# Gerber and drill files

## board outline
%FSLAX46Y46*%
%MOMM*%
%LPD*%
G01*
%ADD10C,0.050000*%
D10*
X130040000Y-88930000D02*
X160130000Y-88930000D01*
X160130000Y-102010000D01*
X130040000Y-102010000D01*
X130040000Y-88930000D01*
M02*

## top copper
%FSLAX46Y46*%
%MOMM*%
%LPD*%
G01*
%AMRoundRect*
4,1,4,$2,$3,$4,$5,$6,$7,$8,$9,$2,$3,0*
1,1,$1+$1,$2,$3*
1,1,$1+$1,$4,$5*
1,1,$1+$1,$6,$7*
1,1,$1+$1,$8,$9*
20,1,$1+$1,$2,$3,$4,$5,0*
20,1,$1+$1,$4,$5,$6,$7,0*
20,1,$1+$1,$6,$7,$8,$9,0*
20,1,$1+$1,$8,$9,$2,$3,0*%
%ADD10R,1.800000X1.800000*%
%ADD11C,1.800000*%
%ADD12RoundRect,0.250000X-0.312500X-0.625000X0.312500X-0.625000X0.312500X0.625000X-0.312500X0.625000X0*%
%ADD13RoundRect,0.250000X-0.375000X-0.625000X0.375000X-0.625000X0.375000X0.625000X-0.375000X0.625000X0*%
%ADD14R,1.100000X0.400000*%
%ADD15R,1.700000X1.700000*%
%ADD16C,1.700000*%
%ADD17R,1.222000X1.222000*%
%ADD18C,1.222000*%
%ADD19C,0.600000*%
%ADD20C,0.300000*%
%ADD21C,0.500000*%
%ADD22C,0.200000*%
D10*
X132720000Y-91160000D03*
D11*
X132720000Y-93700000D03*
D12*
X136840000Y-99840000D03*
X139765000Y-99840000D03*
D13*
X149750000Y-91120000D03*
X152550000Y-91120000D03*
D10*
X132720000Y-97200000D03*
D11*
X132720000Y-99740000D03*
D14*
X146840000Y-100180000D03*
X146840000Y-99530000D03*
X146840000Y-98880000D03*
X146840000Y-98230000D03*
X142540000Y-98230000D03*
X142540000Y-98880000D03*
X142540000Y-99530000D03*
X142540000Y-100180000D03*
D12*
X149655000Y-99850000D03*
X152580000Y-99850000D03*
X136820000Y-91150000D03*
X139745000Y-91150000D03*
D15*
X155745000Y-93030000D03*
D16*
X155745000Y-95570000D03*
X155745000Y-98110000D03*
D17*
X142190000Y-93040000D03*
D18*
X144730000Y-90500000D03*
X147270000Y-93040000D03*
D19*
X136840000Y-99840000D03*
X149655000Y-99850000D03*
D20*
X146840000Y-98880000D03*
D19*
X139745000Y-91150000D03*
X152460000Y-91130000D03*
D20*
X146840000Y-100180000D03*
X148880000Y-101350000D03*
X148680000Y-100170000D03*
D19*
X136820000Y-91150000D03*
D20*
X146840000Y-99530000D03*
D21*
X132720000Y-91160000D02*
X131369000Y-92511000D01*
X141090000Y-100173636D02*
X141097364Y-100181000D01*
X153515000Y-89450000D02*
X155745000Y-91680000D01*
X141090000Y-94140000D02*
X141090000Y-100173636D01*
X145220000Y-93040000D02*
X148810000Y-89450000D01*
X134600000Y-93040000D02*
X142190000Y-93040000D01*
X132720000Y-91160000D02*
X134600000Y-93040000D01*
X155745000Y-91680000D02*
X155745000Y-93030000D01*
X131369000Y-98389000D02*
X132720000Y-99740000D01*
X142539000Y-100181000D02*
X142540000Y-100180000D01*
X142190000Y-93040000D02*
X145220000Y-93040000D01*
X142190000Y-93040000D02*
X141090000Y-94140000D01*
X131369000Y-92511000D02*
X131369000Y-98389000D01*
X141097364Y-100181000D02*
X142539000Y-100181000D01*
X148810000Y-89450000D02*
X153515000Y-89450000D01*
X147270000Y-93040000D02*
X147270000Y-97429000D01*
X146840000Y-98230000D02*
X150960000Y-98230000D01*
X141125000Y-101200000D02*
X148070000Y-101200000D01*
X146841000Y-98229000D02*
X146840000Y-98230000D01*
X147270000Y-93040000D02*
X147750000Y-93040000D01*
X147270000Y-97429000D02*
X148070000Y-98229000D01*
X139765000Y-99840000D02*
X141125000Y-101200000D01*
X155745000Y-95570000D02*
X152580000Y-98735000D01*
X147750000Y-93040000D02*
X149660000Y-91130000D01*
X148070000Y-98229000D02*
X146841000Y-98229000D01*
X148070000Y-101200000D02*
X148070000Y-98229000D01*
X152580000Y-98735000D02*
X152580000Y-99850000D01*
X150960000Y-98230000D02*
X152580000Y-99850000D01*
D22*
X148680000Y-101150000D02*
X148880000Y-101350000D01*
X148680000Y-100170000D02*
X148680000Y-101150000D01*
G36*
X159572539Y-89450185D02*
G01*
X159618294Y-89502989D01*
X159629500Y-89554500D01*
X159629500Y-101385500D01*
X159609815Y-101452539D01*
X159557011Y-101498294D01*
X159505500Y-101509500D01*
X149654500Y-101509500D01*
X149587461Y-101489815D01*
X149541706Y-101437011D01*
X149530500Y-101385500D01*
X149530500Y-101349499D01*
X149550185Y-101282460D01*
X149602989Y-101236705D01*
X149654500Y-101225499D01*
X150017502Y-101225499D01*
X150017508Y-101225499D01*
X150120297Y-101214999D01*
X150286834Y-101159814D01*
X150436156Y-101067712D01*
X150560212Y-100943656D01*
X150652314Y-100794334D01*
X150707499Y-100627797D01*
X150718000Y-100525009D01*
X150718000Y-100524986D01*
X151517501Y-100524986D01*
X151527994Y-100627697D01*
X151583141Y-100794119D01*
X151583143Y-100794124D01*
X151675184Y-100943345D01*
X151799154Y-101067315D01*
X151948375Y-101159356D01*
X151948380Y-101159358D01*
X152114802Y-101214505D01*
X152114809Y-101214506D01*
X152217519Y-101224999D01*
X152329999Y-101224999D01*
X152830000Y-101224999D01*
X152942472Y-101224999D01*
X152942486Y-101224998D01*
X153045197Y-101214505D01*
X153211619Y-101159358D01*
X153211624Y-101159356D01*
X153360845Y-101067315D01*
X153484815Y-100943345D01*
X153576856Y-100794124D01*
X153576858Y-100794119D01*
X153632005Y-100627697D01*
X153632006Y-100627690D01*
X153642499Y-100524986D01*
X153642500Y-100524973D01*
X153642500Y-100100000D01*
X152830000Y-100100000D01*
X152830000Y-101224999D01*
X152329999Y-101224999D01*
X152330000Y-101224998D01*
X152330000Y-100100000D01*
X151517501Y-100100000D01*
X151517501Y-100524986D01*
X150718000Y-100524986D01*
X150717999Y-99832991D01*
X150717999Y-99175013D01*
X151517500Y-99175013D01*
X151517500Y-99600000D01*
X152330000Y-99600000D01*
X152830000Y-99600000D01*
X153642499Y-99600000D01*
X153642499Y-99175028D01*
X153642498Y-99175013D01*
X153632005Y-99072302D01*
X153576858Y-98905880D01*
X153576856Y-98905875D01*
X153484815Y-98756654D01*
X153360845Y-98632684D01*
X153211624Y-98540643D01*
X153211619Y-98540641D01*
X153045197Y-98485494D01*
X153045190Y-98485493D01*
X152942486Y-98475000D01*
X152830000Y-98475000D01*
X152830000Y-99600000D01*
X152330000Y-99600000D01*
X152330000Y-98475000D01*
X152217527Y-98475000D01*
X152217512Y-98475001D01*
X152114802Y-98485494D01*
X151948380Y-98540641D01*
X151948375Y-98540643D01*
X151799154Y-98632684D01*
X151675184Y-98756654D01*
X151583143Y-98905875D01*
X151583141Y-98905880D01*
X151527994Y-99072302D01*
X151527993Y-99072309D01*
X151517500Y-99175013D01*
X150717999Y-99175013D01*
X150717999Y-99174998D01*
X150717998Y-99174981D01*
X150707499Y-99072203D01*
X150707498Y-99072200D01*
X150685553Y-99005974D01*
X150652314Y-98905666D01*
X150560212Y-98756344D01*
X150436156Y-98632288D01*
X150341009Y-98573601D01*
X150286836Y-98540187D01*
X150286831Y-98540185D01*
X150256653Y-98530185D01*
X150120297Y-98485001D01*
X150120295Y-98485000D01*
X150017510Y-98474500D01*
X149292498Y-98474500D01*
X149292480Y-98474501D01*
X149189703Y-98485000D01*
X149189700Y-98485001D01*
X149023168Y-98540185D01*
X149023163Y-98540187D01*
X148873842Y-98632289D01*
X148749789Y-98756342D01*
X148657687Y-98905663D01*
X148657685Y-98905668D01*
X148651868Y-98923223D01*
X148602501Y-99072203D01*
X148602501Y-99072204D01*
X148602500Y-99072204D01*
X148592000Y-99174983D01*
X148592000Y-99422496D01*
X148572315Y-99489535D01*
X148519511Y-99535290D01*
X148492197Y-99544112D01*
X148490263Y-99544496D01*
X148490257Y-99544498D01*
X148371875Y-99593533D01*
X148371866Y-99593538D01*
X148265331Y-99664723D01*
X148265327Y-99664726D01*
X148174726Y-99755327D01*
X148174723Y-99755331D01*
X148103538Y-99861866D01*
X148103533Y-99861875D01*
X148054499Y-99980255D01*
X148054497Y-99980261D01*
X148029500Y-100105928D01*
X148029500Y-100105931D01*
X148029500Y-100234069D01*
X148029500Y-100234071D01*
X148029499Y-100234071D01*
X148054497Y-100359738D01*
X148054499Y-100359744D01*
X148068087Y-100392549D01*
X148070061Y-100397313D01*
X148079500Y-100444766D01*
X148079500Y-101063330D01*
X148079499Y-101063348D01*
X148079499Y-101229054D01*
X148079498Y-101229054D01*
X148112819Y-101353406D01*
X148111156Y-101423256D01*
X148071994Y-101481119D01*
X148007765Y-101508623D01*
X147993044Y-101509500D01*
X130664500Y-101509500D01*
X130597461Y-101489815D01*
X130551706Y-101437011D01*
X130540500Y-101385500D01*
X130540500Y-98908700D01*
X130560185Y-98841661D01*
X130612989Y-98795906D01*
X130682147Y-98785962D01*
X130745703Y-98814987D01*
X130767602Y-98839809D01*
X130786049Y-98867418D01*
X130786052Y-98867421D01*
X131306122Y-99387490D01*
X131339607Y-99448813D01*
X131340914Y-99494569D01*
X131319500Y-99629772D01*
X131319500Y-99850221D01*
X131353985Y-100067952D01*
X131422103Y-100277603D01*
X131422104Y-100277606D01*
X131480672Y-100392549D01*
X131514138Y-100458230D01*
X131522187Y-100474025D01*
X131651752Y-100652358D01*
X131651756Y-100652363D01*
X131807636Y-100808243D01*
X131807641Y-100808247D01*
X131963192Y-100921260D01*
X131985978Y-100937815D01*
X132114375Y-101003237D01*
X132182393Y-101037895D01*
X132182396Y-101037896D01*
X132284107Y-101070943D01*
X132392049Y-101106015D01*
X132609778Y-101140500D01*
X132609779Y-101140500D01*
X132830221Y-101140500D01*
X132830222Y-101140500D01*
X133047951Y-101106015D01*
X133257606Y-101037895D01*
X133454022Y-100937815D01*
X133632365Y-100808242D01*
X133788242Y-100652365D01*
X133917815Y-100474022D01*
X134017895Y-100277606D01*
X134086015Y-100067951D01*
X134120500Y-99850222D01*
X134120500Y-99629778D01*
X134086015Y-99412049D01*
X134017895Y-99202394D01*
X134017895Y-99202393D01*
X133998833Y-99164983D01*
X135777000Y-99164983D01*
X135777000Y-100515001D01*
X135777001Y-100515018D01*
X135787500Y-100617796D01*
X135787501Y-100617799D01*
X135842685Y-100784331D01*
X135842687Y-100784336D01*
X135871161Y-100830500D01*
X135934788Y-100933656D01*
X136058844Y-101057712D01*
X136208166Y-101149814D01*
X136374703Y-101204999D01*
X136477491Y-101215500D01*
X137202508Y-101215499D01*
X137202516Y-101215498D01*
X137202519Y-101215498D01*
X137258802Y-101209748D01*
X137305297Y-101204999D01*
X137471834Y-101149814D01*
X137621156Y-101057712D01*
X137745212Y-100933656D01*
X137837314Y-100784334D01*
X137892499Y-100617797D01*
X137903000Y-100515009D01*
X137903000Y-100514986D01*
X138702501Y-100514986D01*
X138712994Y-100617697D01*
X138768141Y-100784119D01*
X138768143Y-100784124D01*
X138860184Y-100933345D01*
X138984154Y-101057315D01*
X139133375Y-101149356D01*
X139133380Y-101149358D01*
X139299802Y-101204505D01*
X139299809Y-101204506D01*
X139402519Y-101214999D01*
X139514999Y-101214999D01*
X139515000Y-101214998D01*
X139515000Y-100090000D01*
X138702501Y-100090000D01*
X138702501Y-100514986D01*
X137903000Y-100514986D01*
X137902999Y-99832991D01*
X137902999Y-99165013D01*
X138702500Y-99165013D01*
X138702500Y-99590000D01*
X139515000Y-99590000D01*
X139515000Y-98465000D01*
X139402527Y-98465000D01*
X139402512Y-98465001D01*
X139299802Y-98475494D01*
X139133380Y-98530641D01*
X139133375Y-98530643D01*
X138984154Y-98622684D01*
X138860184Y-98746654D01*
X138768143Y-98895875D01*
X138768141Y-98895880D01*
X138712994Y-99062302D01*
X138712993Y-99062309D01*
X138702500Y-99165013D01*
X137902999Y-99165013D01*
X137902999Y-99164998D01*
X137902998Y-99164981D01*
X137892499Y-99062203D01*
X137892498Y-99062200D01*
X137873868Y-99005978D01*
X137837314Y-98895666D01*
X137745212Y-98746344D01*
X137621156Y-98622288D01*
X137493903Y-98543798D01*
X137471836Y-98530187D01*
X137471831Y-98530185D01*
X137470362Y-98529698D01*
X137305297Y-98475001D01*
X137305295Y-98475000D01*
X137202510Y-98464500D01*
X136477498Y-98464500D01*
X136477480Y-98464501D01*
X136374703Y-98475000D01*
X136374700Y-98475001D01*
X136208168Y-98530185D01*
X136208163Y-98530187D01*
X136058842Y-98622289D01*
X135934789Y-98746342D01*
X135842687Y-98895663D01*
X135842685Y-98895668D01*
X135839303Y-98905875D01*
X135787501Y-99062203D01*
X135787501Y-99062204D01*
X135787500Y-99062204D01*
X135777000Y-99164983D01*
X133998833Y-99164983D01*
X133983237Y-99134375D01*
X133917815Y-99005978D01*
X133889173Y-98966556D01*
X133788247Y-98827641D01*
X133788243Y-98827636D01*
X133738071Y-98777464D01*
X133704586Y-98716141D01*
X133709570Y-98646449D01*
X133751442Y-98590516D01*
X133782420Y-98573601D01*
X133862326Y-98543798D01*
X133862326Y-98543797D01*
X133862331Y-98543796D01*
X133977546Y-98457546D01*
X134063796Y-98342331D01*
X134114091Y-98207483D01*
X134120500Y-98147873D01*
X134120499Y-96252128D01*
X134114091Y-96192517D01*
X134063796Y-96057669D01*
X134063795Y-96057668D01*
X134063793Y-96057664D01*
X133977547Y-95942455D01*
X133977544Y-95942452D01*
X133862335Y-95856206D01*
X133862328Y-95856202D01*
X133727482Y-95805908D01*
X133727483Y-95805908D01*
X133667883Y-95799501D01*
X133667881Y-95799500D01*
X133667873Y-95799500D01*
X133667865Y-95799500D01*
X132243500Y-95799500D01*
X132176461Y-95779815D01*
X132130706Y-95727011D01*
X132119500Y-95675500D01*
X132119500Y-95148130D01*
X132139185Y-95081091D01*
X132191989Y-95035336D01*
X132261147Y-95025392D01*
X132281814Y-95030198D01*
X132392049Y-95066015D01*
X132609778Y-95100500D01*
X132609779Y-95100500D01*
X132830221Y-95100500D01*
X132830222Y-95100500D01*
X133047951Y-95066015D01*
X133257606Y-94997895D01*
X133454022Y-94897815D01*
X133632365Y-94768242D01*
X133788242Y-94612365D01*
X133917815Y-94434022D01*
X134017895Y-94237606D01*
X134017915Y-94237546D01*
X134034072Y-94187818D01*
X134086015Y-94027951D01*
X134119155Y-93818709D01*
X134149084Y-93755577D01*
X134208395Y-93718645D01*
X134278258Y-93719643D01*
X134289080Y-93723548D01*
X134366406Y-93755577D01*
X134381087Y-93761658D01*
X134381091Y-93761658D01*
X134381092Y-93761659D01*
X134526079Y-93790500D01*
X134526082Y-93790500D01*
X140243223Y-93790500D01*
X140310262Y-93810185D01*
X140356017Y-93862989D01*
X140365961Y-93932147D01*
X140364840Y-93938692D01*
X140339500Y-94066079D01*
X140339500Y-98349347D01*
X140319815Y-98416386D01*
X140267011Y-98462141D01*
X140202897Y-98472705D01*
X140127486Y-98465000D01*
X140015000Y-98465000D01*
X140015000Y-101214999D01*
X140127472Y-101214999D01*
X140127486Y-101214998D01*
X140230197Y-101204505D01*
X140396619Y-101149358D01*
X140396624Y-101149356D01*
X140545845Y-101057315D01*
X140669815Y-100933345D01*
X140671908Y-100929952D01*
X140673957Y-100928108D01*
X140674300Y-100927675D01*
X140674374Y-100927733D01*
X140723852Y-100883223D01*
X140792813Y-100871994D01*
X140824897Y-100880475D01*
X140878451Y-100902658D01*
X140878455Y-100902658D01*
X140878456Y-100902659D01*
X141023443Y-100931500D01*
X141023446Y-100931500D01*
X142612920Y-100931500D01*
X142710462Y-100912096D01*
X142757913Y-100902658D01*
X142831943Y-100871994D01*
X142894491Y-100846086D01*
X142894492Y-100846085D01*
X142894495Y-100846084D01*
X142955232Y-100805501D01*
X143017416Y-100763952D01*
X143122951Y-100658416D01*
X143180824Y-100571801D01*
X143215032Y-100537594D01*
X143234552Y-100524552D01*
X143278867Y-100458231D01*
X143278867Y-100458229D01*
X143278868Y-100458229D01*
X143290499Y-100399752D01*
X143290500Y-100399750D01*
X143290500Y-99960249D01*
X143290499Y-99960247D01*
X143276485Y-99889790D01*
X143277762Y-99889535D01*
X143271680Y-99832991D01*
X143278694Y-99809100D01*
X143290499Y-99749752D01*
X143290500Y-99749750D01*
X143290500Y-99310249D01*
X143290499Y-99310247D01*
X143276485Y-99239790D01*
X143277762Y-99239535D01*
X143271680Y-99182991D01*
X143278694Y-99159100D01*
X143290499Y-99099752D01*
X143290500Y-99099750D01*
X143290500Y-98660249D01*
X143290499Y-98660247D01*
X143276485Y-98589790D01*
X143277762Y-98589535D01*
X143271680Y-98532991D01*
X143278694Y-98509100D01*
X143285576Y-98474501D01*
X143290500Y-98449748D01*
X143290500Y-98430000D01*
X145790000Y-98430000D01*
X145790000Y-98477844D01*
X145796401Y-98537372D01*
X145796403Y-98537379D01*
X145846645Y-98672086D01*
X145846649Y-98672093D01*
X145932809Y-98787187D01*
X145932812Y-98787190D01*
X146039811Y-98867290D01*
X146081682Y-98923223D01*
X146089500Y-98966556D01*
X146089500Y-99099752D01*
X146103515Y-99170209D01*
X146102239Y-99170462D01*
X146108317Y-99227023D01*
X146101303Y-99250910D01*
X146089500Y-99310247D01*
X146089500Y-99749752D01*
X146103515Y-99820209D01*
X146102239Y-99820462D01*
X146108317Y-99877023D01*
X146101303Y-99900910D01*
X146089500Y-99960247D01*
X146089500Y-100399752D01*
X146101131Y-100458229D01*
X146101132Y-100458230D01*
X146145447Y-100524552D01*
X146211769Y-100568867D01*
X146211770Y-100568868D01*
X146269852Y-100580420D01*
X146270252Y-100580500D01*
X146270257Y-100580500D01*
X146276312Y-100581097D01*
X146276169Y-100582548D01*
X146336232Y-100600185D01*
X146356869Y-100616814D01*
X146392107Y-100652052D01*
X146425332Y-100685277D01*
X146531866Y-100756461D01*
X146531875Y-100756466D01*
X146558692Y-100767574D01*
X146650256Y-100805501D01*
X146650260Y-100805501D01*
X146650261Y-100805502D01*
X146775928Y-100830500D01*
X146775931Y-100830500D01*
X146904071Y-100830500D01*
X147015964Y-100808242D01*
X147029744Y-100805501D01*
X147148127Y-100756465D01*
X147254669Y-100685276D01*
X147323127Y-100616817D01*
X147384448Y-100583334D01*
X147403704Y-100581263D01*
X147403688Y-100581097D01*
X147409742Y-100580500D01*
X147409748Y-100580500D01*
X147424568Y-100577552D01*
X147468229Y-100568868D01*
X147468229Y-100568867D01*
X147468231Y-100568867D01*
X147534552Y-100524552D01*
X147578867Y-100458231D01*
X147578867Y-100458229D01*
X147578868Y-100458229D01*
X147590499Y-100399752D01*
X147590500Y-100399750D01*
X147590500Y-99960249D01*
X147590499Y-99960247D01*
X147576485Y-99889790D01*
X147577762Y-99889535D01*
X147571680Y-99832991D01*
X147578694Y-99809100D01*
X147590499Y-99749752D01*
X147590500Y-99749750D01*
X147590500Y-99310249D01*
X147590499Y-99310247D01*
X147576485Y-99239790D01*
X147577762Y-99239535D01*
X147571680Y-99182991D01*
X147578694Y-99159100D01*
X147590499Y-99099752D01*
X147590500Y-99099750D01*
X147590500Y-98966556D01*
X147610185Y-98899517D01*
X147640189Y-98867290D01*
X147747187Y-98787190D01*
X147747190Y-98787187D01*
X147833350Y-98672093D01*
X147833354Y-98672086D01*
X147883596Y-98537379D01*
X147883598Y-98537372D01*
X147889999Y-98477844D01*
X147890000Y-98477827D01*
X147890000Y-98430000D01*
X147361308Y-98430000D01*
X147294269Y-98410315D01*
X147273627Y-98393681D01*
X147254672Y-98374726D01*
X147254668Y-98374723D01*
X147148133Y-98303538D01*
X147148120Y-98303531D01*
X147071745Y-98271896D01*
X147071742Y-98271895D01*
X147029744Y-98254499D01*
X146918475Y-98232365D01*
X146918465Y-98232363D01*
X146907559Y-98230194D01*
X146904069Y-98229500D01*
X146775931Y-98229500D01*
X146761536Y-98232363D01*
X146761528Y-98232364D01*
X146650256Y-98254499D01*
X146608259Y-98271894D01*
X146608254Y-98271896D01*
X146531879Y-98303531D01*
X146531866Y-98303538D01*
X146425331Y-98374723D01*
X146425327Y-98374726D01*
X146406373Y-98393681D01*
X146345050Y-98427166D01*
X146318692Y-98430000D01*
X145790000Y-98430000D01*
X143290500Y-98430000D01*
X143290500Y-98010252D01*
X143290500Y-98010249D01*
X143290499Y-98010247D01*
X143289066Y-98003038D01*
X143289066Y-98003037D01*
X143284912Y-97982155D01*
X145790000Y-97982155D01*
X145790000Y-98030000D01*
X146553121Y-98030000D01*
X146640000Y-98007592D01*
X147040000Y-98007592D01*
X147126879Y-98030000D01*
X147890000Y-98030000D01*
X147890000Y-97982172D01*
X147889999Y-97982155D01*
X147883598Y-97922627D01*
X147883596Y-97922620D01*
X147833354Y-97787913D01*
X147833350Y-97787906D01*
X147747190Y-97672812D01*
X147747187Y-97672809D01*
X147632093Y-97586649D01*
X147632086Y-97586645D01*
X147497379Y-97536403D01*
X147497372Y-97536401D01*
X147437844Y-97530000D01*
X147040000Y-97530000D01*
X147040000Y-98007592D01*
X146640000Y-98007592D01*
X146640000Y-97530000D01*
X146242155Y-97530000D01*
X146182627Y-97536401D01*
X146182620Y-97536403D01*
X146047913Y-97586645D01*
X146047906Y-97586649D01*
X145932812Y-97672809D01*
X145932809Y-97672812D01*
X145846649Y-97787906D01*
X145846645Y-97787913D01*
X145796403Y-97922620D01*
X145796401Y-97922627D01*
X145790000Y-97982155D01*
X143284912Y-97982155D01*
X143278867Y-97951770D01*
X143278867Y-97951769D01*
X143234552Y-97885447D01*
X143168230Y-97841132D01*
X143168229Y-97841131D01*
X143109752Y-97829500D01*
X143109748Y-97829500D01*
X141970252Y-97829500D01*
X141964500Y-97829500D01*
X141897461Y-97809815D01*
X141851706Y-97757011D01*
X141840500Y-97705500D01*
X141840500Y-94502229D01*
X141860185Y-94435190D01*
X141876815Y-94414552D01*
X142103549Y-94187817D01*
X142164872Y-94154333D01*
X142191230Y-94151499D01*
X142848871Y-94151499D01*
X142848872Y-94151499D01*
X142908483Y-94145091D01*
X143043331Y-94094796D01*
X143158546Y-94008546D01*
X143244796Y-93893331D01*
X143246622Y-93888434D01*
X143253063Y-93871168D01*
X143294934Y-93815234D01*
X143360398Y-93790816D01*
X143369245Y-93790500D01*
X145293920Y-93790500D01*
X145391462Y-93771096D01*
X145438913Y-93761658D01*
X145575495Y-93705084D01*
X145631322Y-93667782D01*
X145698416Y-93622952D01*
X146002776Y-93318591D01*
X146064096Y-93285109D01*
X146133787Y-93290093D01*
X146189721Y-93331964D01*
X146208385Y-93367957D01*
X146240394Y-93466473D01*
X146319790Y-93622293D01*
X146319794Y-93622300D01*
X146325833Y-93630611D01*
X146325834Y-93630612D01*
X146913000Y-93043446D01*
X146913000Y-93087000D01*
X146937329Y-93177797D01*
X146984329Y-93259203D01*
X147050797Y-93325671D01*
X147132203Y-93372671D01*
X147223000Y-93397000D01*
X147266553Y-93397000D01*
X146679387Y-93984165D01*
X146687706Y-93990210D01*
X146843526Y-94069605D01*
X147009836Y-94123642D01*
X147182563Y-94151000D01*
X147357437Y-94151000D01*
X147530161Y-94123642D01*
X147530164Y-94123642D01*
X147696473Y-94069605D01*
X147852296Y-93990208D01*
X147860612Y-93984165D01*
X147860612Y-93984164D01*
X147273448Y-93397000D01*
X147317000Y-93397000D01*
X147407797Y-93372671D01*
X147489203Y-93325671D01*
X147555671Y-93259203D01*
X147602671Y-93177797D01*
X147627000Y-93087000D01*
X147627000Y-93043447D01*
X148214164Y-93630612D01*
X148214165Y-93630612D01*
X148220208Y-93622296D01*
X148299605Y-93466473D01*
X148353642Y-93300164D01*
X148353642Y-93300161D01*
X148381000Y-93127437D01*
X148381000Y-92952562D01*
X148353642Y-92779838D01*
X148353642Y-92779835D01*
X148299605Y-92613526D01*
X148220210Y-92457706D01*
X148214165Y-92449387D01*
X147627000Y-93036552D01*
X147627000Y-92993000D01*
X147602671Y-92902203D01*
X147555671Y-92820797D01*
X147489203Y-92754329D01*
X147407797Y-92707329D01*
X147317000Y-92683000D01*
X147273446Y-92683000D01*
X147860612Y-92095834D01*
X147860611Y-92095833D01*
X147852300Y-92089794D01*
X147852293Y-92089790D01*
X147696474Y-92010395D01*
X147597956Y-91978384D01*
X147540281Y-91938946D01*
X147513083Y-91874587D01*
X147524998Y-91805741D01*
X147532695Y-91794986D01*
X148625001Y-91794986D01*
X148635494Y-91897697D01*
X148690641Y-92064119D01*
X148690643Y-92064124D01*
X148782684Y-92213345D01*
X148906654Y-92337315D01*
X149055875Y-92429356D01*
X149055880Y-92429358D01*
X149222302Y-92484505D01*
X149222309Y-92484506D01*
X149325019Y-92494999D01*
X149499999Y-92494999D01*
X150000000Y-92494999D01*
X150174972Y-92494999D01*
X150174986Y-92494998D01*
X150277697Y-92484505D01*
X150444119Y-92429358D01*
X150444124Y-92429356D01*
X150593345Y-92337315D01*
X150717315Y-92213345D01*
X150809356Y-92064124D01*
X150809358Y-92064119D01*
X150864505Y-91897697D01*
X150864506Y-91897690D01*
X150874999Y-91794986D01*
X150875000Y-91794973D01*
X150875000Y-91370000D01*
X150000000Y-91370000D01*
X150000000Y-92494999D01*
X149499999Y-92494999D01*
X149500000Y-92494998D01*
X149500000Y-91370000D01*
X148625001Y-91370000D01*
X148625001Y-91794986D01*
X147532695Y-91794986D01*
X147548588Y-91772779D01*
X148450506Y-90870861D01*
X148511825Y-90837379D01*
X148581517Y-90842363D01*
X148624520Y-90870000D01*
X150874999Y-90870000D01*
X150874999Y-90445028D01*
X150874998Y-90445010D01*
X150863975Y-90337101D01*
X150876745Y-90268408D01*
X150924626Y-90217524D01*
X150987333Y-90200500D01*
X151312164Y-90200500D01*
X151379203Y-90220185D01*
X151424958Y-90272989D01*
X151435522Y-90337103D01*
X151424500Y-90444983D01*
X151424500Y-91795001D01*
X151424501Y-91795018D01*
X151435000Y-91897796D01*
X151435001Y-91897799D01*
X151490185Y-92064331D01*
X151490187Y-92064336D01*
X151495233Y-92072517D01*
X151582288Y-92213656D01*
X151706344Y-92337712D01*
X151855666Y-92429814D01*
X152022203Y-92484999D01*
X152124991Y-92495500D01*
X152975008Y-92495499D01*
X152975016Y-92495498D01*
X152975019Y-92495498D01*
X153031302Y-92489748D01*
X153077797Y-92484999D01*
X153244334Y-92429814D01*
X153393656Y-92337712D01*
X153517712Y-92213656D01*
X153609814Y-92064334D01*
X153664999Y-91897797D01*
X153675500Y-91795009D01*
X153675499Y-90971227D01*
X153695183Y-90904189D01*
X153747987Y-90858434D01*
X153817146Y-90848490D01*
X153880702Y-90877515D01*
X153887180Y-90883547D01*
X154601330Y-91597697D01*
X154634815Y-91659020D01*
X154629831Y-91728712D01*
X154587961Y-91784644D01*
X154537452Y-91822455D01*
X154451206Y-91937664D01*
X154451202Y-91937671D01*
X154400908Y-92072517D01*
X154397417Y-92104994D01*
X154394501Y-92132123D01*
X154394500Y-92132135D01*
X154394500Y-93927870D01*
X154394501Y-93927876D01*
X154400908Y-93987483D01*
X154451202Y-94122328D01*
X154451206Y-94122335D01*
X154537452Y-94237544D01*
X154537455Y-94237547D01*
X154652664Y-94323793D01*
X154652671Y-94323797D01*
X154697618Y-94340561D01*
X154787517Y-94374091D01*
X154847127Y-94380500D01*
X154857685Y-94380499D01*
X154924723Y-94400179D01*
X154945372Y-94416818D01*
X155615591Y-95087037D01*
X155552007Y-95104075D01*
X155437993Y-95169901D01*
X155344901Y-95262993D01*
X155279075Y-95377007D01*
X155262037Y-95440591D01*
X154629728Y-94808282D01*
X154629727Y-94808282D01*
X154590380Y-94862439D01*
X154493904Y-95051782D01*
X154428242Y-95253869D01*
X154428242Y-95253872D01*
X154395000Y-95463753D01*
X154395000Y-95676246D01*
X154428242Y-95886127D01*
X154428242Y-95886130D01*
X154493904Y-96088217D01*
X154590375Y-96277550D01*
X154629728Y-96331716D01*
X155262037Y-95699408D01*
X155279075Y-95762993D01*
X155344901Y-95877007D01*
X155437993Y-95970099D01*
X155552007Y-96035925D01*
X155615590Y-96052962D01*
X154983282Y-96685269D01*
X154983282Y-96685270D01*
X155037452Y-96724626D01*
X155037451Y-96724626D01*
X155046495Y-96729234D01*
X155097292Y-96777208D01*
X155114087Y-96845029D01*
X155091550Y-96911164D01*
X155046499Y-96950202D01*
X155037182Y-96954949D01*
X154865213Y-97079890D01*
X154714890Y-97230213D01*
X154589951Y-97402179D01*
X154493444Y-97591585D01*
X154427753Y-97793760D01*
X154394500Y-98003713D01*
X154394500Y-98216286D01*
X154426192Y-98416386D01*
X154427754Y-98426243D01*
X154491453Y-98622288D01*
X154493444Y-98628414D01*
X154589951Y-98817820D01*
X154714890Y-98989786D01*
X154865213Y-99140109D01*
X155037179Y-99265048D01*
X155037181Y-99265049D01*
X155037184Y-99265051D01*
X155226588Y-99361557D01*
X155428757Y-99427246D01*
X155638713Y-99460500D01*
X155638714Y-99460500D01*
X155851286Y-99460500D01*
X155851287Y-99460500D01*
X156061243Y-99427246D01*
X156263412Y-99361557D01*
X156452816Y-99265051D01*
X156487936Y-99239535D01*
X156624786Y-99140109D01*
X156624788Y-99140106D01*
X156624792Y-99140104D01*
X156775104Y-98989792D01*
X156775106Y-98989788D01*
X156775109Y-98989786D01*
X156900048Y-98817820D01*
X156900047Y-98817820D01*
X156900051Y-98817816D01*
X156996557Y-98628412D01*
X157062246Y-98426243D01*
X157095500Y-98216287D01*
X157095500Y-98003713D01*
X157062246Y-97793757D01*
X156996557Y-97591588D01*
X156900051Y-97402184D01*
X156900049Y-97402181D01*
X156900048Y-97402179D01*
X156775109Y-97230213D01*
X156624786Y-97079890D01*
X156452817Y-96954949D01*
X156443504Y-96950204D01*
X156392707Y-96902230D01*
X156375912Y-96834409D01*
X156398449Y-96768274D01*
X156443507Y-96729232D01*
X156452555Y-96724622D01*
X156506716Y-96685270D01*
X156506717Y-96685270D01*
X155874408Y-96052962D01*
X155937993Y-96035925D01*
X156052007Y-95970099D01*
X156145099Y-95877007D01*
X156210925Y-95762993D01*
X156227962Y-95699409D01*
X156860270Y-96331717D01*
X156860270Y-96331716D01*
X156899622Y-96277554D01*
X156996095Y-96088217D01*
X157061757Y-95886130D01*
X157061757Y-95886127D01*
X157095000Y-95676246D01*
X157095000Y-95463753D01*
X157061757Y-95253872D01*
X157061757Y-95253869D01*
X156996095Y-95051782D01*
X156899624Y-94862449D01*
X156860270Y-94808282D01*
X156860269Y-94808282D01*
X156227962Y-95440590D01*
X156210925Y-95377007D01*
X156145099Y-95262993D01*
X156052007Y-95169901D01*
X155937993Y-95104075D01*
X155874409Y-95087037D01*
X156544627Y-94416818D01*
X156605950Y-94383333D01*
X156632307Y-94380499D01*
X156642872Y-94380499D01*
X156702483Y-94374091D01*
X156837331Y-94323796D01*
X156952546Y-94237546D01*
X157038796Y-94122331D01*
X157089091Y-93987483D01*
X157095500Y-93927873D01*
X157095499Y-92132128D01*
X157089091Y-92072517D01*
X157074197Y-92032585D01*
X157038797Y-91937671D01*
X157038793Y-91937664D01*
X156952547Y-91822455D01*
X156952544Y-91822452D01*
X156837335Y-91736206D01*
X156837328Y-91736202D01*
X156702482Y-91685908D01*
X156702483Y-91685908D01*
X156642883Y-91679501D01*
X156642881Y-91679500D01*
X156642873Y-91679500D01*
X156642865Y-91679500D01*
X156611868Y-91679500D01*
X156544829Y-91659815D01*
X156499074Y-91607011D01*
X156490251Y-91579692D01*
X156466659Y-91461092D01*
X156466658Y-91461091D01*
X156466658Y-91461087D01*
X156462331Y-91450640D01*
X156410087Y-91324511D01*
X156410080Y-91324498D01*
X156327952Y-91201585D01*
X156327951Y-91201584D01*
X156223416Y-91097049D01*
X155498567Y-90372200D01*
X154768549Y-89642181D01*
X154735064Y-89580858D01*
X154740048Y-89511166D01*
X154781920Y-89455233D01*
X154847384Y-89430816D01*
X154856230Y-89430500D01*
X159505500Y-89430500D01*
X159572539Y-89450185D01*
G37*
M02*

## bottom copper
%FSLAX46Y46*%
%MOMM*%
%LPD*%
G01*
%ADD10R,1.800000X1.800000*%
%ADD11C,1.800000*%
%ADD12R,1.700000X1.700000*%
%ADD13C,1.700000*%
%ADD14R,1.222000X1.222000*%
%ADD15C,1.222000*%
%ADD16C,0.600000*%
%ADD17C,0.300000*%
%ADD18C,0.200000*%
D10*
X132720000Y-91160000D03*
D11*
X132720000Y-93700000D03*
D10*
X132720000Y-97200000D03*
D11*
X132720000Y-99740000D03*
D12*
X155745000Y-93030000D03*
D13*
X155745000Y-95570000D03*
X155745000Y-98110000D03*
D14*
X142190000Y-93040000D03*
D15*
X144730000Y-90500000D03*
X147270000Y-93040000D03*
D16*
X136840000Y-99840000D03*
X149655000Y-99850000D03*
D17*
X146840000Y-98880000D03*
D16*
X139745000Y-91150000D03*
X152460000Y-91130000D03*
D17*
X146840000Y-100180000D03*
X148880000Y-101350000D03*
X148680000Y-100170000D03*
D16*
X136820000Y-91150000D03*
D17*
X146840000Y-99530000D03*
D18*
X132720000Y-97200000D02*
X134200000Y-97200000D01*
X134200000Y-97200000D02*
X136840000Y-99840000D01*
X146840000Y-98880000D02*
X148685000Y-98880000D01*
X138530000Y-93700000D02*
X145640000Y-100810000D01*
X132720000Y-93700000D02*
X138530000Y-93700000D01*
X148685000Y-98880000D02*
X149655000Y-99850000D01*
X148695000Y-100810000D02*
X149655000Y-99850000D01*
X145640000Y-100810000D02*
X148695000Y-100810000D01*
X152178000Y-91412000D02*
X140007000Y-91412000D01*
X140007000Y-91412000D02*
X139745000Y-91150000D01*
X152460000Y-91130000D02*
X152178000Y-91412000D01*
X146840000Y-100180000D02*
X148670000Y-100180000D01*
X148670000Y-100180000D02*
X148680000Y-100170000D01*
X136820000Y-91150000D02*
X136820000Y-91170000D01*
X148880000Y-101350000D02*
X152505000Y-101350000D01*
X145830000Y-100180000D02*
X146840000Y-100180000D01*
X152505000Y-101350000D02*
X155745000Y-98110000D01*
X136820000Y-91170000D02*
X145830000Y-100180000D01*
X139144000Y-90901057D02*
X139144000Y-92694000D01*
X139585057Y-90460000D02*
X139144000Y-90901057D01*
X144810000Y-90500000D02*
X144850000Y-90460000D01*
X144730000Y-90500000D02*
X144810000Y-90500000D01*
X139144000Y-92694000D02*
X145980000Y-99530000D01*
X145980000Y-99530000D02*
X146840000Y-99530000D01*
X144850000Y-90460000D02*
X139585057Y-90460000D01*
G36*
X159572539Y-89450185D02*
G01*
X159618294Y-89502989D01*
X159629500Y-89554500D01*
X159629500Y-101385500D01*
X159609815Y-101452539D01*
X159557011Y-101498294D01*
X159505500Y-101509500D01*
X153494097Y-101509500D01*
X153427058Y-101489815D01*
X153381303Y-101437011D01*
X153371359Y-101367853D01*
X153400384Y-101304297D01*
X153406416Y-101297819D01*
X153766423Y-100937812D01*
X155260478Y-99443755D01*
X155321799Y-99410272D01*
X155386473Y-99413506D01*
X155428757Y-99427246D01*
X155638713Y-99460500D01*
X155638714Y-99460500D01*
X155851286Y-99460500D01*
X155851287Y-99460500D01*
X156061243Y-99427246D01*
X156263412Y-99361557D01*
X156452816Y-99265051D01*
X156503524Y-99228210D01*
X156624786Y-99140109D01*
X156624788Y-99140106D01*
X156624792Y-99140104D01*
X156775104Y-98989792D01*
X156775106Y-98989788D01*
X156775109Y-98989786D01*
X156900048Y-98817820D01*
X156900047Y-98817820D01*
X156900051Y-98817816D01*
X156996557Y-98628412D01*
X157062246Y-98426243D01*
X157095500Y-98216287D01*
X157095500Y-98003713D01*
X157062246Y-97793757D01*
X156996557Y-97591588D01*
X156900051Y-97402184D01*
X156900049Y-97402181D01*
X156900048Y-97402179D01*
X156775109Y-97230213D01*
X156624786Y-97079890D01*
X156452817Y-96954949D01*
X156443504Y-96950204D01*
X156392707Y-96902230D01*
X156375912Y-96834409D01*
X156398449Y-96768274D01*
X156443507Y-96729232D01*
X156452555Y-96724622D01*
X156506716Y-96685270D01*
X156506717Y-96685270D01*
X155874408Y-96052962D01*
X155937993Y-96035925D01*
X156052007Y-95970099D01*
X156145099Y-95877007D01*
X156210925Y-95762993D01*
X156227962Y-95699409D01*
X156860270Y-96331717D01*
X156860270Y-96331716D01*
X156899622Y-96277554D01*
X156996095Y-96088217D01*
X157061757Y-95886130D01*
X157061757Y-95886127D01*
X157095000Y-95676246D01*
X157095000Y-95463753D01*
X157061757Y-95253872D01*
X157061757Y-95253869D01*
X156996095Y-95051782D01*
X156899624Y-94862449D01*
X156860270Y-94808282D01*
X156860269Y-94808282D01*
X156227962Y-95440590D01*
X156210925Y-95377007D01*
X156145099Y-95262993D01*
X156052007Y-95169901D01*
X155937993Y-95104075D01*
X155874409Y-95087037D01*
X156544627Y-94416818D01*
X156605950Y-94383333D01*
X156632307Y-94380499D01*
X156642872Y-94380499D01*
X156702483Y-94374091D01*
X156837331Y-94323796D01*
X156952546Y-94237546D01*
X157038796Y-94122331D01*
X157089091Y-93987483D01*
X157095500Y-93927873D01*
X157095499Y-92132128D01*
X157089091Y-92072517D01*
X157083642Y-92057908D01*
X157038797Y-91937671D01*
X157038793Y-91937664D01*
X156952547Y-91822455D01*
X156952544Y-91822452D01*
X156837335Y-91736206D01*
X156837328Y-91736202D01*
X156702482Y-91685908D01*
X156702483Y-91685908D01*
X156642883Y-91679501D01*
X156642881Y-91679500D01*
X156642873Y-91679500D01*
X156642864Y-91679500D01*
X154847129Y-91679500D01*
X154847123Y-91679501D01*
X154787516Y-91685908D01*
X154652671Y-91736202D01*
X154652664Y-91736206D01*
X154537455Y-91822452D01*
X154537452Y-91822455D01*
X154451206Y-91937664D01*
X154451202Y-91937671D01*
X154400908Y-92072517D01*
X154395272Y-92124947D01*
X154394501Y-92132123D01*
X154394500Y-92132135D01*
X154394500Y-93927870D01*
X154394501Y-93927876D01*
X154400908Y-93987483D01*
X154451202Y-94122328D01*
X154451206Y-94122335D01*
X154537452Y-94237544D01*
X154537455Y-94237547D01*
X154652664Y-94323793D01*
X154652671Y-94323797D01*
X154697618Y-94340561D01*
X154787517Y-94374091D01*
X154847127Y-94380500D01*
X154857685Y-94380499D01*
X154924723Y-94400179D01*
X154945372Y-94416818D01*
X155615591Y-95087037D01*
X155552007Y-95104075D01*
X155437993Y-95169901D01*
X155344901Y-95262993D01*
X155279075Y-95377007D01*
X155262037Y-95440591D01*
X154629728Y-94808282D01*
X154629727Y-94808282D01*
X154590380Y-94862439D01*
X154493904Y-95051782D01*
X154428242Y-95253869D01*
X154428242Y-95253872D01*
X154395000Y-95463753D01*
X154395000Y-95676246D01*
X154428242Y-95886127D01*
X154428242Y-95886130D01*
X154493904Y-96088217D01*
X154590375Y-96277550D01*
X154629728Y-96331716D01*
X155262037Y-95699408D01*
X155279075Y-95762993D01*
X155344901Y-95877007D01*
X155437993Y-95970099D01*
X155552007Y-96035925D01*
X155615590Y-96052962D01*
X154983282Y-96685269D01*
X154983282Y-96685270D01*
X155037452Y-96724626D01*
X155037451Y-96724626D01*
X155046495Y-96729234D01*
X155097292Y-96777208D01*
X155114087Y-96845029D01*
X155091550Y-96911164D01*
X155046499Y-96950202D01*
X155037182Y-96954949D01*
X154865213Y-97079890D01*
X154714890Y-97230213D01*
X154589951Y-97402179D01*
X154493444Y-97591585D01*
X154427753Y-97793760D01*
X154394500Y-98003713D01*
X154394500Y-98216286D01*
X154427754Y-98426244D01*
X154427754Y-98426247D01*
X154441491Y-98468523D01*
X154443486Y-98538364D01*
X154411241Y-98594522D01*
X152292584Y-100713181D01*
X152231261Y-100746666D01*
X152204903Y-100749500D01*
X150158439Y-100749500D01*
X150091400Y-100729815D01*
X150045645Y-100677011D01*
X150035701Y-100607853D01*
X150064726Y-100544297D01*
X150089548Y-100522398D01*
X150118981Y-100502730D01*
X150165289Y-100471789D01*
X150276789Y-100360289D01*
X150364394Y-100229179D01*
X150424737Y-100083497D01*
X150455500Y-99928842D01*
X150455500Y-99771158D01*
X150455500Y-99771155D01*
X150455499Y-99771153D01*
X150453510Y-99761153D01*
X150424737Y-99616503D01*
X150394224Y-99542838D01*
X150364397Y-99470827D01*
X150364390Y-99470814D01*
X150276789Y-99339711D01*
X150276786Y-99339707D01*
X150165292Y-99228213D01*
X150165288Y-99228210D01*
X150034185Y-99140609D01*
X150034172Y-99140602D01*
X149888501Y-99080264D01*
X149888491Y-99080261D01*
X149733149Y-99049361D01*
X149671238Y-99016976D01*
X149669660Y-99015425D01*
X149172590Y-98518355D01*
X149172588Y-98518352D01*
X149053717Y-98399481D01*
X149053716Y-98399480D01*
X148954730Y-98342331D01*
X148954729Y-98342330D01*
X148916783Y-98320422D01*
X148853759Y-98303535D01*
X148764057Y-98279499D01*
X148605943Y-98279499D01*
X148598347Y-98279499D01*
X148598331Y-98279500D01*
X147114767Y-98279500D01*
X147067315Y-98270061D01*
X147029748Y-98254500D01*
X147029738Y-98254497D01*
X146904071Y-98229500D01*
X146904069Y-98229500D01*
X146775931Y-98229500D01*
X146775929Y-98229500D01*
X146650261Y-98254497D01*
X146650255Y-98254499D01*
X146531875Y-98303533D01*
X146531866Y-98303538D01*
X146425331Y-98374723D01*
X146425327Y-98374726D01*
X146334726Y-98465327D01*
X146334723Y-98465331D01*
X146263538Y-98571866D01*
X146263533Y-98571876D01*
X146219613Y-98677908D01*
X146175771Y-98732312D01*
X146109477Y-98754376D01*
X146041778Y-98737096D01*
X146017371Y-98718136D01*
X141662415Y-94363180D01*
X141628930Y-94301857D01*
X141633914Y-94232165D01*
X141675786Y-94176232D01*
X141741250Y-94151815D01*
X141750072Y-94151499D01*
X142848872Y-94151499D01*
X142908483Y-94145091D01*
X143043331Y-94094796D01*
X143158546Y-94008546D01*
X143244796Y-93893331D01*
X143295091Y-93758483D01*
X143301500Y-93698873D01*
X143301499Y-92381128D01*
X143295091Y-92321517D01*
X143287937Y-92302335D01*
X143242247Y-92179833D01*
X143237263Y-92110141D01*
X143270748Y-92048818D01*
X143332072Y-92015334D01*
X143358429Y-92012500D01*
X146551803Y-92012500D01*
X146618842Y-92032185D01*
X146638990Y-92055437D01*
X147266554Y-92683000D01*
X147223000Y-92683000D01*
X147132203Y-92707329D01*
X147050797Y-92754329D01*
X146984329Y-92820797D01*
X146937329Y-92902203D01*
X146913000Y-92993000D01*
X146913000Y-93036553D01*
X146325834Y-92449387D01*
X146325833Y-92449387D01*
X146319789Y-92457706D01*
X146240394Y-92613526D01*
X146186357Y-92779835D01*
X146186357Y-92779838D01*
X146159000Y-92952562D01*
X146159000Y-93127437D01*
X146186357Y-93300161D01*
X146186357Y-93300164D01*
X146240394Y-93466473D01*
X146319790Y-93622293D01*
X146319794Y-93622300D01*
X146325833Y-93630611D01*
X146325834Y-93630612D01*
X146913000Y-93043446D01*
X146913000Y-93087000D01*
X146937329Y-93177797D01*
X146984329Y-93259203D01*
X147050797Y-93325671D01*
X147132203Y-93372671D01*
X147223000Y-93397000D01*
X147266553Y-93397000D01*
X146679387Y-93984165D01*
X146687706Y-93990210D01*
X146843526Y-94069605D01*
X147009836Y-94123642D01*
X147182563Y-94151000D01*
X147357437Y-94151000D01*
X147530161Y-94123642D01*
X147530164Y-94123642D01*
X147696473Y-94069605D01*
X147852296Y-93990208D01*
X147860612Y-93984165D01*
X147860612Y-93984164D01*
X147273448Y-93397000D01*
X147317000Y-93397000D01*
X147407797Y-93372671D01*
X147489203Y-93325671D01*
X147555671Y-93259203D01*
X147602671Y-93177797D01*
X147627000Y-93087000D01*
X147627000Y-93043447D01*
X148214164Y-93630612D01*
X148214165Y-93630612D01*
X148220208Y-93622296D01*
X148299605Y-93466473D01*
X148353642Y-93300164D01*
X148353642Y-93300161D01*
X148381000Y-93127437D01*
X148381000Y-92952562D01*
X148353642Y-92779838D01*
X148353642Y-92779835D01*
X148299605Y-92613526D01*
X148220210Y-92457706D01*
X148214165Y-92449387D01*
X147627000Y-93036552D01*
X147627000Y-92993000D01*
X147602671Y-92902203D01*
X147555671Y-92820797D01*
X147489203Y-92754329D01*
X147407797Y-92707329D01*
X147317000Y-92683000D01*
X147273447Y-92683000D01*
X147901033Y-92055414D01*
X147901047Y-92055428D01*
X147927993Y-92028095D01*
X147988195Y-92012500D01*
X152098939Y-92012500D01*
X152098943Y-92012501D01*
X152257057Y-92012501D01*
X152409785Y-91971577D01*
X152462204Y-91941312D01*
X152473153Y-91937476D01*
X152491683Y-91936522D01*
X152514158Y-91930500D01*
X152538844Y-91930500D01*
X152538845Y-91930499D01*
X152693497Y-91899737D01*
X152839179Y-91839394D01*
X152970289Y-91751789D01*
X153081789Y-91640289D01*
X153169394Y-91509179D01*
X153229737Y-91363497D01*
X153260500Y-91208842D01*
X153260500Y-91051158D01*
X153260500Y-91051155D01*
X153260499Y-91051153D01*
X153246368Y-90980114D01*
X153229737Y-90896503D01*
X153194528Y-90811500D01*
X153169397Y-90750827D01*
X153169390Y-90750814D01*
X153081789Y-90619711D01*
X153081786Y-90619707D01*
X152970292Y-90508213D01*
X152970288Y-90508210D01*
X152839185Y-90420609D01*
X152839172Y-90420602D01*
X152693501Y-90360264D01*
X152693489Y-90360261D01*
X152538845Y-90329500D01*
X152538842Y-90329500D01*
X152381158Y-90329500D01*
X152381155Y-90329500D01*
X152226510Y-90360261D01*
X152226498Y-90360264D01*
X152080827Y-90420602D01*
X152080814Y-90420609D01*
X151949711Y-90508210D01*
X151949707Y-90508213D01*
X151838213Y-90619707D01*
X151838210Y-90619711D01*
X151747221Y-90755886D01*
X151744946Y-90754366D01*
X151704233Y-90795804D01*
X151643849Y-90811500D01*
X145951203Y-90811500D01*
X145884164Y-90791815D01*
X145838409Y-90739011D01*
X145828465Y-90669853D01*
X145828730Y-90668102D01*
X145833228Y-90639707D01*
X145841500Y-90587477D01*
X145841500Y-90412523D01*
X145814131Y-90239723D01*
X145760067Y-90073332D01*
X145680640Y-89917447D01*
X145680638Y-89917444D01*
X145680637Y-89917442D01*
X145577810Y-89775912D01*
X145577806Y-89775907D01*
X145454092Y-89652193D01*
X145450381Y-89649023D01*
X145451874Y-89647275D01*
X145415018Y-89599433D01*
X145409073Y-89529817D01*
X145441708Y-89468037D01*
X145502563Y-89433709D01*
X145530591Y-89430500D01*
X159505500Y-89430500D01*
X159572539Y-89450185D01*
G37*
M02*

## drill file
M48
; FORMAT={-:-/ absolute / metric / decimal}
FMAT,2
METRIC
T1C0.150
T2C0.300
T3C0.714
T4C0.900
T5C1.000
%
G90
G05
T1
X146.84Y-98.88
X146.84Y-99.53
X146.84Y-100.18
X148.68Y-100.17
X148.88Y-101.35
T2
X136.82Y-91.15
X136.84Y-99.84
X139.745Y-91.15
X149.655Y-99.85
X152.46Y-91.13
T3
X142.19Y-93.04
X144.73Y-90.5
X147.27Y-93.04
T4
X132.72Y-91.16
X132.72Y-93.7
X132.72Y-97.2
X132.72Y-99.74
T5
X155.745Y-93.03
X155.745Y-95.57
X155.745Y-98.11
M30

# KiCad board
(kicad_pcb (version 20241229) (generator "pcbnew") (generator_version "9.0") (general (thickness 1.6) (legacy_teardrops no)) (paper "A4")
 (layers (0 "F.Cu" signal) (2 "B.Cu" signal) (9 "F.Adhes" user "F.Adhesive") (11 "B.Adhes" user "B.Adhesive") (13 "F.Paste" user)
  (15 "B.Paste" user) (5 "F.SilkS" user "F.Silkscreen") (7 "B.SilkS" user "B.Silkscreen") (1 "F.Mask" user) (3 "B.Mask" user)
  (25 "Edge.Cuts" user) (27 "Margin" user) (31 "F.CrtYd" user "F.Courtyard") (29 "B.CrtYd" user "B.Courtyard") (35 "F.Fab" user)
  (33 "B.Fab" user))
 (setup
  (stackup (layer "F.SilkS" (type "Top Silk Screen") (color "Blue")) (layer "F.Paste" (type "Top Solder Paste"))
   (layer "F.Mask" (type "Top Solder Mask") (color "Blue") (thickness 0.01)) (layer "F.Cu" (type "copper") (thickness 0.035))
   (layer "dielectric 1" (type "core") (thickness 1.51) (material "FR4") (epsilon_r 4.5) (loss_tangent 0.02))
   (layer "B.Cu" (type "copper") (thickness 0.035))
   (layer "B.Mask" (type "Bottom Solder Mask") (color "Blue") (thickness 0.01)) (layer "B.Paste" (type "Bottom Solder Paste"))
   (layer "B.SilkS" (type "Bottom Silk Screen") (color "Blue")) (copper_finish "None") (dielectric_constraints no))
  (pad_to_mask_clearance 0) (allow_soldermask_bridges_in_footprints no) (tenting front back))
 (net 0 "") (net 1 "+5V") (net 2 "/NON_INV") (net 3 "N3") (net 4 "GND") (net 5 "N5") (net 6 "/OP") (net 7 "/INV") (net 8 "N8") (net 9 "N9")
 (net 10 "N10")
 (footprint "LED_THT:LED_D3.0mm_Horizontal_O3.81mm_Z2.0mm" (layer "F.Cu") (at 132.72 91.16 -90)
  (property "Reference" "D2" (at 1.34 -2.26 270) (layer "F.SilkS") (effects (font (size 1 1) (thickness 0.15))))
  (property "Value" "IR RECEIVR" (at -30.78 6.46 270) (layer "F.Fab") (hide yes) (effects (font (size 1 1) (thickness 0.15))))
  (pad "1" thru_hole rect (at 0 0 270) (size 1.8 1.8) (drill 0.9) (layers "*.Cu" "*.Mask") (remove_unused_layers no) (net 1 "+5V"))
  (pad "2" thru_hole circle (at 2.54 0 270) (size 1.8 1.8) (drill 0.9) (layers "*.Cu" "*.Mask") (remove_unused_layers no) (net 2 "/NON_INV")))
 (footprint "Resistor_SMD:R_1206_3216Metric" (layer "F.Cu") (at 138.3025 99.84)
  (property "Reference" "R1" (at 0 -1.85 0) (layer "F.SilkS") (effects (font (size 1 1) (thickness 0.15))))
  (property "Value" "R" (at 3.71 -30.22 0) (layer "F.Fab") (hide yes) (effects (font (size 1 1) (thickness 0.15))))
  (pad "1" smd roundrect (at -1.4625 0) (size 1.125 1.75) (layers "F.Cu" "F.Mask" "F.Paste") (roundrect_rratio 0.222222) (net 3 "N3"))
  (pad "2" smd roundrect (at 1.4625 0) (size 1.125 1.75) (layers "F.Cu" "F.Mask" "F.Paste") (roundrect_rratio 0.222222) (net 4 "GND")))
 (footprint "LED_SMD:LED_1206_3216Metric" (layer "F.Cu") (at 151.15 91.12)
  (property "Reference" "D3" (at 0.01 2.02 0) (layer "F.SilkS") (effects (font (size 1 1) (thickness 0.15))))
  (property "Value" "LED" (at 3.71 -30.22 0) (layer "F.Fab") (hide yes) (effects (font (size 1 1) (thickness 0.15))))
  (pad "1" smd roundrect (at -1.4 0) (size 1.25 1.75) (layers "F.Cu" "F.Mask" "F.Paste") (roundrect_rratio 0.2) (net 4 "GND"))
  (pad "2" smd roundrect (at 1.4 0) (size 1.25 1.75) (layers "F.Cu" "F.Mask" "F.Paste") (roundrect_rratio 0.2) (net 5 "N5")))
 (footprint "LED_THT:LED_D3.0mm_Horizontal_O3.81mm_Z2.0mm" (layer "F.Cu") (at 132.72 97.2 -90)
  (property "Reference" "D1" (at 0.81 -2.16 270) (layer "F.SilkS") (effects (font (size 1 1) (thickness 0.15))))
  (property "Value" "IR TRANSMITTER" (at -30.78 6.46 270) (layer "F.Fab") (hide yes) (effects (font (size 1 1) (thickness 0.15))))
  (pad "1" thru_hole rect (at 0 0 270) (size 1.8 1.8) (drill 0.9) (layers "*.Cu" "*.Mask") (remove_unused_layers no) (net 3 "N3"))
  (pad "2" thru_hole circle (at 2.54 0 270) (size 1.8 1.8) (drill 0.9) (layers "*.Cu" "*.Mask") (remove_unused_layers no) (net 1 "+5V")))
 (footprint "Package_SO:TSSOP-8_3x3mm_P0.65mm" (layer "F.Cu") (at 144.69 99.205 180)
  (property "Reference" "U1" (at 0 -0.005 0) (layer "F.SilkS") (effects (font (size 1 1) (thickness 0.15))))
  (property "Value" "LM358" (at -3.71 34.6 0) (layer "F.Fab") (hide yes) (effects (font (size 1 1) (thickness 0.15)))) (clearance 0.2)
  (pad "1" smd rect (at -2.15 -0.975 180) (size 1.1 0.4) (layers "F.Cu" "F.Mask" "F.Paste") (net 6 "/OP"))
  (pad "2" smd rect (at -2.15 -0.325 180) (size 1.1 0.4) (layers "F.Cu" "F.Mask" "F.Paste") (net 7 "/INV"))
  (pad "3" smd rect (at -2.15 0.325 180) (size 1.1 0.4) (layers "F.Cu" "F.Mask" "F.Paste") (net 2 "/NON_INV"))
  (pad "4" smd rect (at -2.15 0.975 180) (size 1.1 0.4) (layers "F.Cu" "F.Mask" "F.Paste") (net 4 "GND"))
  (pad "5" smd rect (at 2.15 0.975 180) (size 1.1 0.4) (layers "F.Cu" "F.Mask" "F.Paste") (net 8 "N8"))
  (pad "6" smd rect (at 2.15 0.325 180) (size 1.1 0.4) (layers "F.Cu" "F.Mask" "F.Paste") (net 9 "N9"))
  (pad "7" smd rect (at 2.15 -0.325 180) (size 1.1 0.4) (layers "F.Cu" "F.Mask" "F.Paste") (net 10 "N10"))
  (pad "8" smd rect (at 2.15 -0.975 180) (size 1.1 0.4) (layers "F.Cu" "F.Mask" "F.Paste") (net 1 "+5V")))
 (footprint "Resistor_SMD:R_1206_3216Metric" (layer "F.Cu") (at 151.1175 99.85)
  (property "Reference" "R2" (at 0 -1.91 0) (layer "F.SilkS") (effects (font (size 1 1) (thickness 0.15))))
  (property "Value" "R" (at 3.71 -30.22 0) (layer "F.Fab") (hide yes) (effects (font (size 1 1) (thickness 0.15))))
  (pad "1" smd roundrect (at -1.4625 0) (size 1.125 1.75) (layers "F.Cu" "F.Mask" "F.Paste") (roundrect_rratio 0.222222) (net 2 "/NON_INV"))
  (pad "2" smd roundrect (at 1.4625 0) (size 1.125 1.75) (layers "F.Cu" "F.Mask" "F.Paste") (roundrect_rratio 0.222222) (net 4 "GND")))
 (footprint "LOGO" (layer "F.Cu") (at 151.112918 95.427453)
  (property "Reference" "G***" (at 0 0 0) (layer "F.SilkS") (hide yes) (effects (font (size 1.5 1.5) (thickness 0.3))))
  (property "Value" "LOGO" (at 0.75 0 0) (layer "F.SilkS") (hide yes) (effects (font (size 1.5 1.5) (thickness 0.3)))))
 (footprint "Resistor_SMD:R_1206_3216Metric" (layer "F.Cu") (at 138.2825 91.15)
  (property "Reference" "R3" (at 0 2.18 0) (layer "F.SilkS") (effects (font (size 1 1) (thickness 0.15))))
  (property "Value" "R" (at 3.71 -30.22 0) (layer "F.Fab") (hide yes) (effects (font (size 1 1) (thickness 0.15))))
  (pad "1" smd roundrect (at -1.4625 0) (size 1.125 1.75) (layers "F.Cu" "F.Mask" "F.Paste") (roundrect_rratio 0.222222) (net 6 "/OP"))
  (pad "2" smd roundrect (at 1.4625 0) (size 1.125 1.75) (layers "F.Cu" "F.Mask" "F.Paste") (roundrect_rratio 0.222222) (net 5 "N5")))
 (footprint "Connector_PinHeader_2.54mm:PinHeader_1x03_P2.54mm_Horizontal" (layer "F.Cu") (at 155.745 93.03)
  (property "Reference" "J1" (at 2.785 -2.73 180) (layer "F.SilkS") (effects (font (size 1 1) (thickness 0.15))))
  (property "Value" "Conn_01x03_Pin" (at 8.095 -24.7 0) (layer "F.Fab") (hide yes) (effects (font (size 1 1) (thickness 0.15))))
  (pad "1" thru_hole rect (at 0 0) (size 1.7 1.7) (drill 1) (layers "*.Cu" "*.Mask") (remove_unused_layers no) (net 1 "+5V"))
  (pad "2" thru_hole circle (at 0 2.54) (size 1.7 1.7) (drill 1) (layers "*.Cu" "*.Mask") (remove_unused_layers no) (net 4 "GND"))
  (pad "3" thru_hole circle (at 0 5.08) (size 1.7 1.7) (drill 1) (layers "*.Cu" "*.Mask") (remove_unused_layers no) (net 6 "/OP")))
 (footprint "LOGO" (layer "F.Cu") (at 138.1 95.605825)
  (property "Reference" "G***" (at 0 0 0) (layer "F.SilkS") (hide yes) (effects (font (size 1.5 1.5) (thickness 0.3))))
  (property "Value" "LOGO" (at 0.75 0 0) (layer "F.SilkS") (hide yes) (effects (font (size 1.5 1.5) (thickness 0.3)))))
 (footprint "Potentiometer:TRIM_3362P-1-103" (layer "F.Cu") (at 144.73 93.04)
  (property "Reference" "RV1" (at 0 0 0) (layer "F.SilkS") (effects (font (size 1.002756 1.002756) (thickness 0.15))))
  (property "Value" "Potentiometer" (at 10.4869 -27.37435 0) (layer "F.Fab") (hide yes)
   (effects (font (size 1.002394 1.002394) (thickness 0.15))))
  (pad "1" thru_hole rect (at -2.54 0) (size 1.222 1.222) (drill 0.714) (layers "*.Cu" "*.Mask") (remove_unused_layers no) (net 1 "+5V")
   (solder_mask_margin 0.102))
  (pad "2" thru_hole circle (at 0 -2.54) (size 1.222 1.222) (drill 0.714) (layers "*.Cu" "*.Mask") (remove_unused_layers no) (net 7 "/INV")
   (solder_mask_margin 0.102))
  (pad "3" thru_hole circle (at 2.54 0) (size 1.222 1.222) (drill 0.714) (layers "*.Cu" "*.Mask") (remove_unused_layers no) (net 4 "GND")
   (solder_mask_margin 0.102)))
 (gr_rect (start 130.04 88.93) (end 160.13 102.01) (stroke (width 0.05) (type default)) (fill no) (layer "Edge.Cuts"))
 (segment (start 132.72 91.16) (end 131.369 92.511) (width 0.5) (layer "F.Cu") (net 1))
 (segment (start 141.09 100.173636) (end 141.097364 100.181) (width 0.5) (layer "F.Cu") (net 1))
 (segment (start 153.515 89.45) (end 155.745 91.68) (width 0.5) (layer "F.Cu") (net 1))
 (segment (start 141.09 94.14) (end 141.09 100.173636) (width 0.5) (layer "F.Cu") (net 1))
 (segment (start 145.22 93.04) (end 148.81 89.45) (width 0.5) (layer "F.Cu") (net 1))
 (segment (start 134.6 93.04) (end 142.19 93.04) (width 0.5) (layer "F.Cu") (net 1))
 (segment (start 132.72 91.16) (end 134.6 93.04) (width 0.5) (layer "F.Cu") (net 1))
 (segment (start 155.745 91.68) (end 155.745 93.03) (width 0.5) (layer "F.Cu") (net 1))
 (segment (start 131.369 98.389) (end 132.72 99.74) (width 0.5) (layer "F.Cu") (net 1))
 (segment (start 142.539 100.181) (end 142.54 100.18) (width 0.5) (layer "F.Cu") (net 1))
 (segment (start 142.19 93.04) (end 145.22 93.04) (width 0.5) (layer "F.Cu") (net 1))
 (segment (start 142.19 93.04) (end 141.09 94.14) (width 0.5) (layer "F.Cu") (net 1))
 (segment (start 131.369 92.511) (end 131.369 98.389) (width 0.5) (layer "F.Cu") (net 1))
 (segment (start 141.097364 100.181) (end 142.539 100.181) (width 0.5) (layer "F.Cu") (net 1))
 (segment (start 148.81 89.45) (end 153.515 89.45) (width 0.5) (layer "F.Cu") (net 1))
 (via (at 136.84 99.84) (size 0.6) (drill 0.3) (layers "F.Cu" "B.Cu") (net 3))
 (segment (start 132.72 97.2) (end 134.2 97.2) (width 0.2) (layer "B.Cu") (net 3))
 (segment (start 134.2 97.2) (end 136.84 99.84) (width 0.2) (layer "B.Cu") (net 3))
 (via (at 149.655 99.85) (size 0.6) (drill 0.3) (layers "F.Cu" "B.Cu") (free yes) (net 2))
 (via (at 146.84 98.88) (size 0.3) (drill 0.15) (layers "F.Cu" "B.Cu") (free yes) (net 2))
 (segment (start 146.84 98.88) (end 148.685 98.88) (width 0.2) (layer "B.Cu") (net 2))
 (segment (start 138.53 93.7) (end 145.64 100.81) (width 0.2) (layer "B.Cu") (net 2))
 (segment (start 132.72 93.7) (end 138.53 93.7) (width 0.2) (layer "B.Cu") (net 2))
 (segment (start 148.685 98.88) (end 149.655 99.85) (width 0.2) (layer "B.Cu") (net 2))
 (segment (start 148.695 100.81) (end 149.655 99.85) (width 0.2) (layer "B.Cu") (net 2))
 (segment (start 145.64 100.81) (end 148.695 100.81) (width 0.2) (layer "B.Cu") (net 2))
 (segment (start 147.27 93.04) (end 147.27 97.429) (width 0.5) (layer "F.Cu") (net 4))
 (segment (start 146.84 98.23) (end 150.96 98.23) (width 0.5) (layer "F.Cu") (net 4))
 (segment (start 141.125 101.2) (end 148.07 101.2) (width 0.5) (layer "F.Cu") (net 4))
 (segment (start 146.841 98.229) (end 146.84 98.23) (width 0.5) (layer "F.Cu") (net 4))
 (segment (start 147.27 93.04) (end 147.75 93.04) (width 0.5) (layer "F.Cu") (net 4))
 (segment (start 147.27 97.429) (end 148.07 98.229) (width 0.5) (layer "F.Cu") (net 4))
 (segment (start 139.765 99.84) (end 141.125 101.2) (width 0.5) (layer "F.Cu") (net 4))
 (segment (start 155.745 95.57) (end 152.58 98.735) (width 0.5) (layer "F.Cu") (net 4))
 (segment (start 147.75 93.04) (end 149.66 91.13) (width 0.5) (layer "F.Cu") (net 4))
 (segment (start 148.07 98.229) (end 146.841 98.229) (width 0.5) (layer "F.Cu") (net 4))
 (segment (start 148.07 101.2) (end 148.07 98.229) (width 0.5) (layer "F.Cu") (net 4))
 (segment (start 152.58 98.735) (end 152.58 99.85) (width 0.5) (layer "F.Cu") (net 4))
 (segment (start 150.96 98.23) (end 152.58 99.85) (width 0.5) (layer "F.Cu") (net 4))
 (via (at 139.745 91.15) (size 0.6) (drill 0.3) (layers "F.Cu" "B.Cu") (free yes) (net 5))
 (via (at 152.46 91.13) (size 0.6) (drill 0.3) (layers "F.Cu" "B.Cu") (free yes) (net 5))
 (segment (start 152.178 91.412) (end 140.007 91.412) (width 0.2) (layer "B.Cu") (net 5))
 (segment (start 140.007 91.412) (end 139.745 91.15) (width 0.2) (layer "B.Cu") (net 5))
 (segment (start 152.46 91.13) (end 152.178 91.412) (width 0.2) (layer "B.Cu") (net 5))
 (segment (start 148.68 101.15) (end 148.88 101.35) (width 0.2) (layer "F.Cu") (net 6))
 (segment (start 148.68 100.17) (end 148.68 101.15) (width 0.2) (layer "F.Cu") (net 6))
 (via (at 146.84 100.18) (size 0.3) (drill 0.15) (layers "F.Cu" "B.Cu") (free yes) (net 6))
 (via (at 148.88 101.35) (size 0.3) (drill 0.15) (layers "F.Cu" "B.Cu") (free yes) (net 6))
 (via (at 148.68 100.17) (size 0.3) (drill 0.15) (layers "F.Cu" "B.Cu") (free yes) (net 6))
 (via (at 136.82 91.15) (size 0.6) (drill 0.3) (layers "F.Cu" "B.Cu") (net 6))
 (segment (start 146.84 100.18) (end 148.67 100.18) (width 0.2) (layer "B.Cu") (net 6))
 (segment (start 148.67 100.18) (end 148.68 100.17) (width 0.2) (layer "B.Cu") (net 6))
 (segment (start 136.82 91.15) (end 136.82 91.17) (width 0.2) (layer "B.Cu") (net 6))
 (segment (start 148.88 101.35) (end 152.505 101.35) (width 0.2) (layer "B.Cu") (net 6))
 (segment (start 145.83 100.18) (end 146.84 100.18) (width 0.2) (layer "B.Cu") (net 6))
 (segment (start 152.505 101.35) (end 155.745 98.11) (width 0.2) (layer "B.Cu") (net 6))
 (segment (start 136.82 91.17) (end 145.83 100.18) (width 0.2) (layer "B.Cu") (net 6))
 (via (at 146.84 99.53) (size 0.3) (drill 0.15) (layers "F.Cu" "B.Cu") (free yes) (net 7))
 (segment (start 139.144 90.901057) (end 139.144 92.694) (width 0.2) (layer "B.Cu") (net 7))
 (segment (start 139.585057 90.46) (end 139.144 90.901057) (width 0.2) (layer "B.Cu") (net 7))
 (segment (start 144.81 90.5) (end 144.85 90.46) (width 0.2) (layer "B.Cu") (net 7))
 (segment (start 144.73 90.5) (end 144.81 90.5) (width 0.2) (layer "B.Cu") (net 7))
 (segment (start 139.144 92.694) (end 145.98 99.53) (width 0.2) (layer "B.Cu") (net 7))
 (segment (start 145.98 99.53) (end 146.84 99.53) (width 0.2) (layer "B.Cu") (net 7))
 (segment (start 144.85 90.46) (end 139.585057 90.46) (width 0.2) (layer "B.Cu") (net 7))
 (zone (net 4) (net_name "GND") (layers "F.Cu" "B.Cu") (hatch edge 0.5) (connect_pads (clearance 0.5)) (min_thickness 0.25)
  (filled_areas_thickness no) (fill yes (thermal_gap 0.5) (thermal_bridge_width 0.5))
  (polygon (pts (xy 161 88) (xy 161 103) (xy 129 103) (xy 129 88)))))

